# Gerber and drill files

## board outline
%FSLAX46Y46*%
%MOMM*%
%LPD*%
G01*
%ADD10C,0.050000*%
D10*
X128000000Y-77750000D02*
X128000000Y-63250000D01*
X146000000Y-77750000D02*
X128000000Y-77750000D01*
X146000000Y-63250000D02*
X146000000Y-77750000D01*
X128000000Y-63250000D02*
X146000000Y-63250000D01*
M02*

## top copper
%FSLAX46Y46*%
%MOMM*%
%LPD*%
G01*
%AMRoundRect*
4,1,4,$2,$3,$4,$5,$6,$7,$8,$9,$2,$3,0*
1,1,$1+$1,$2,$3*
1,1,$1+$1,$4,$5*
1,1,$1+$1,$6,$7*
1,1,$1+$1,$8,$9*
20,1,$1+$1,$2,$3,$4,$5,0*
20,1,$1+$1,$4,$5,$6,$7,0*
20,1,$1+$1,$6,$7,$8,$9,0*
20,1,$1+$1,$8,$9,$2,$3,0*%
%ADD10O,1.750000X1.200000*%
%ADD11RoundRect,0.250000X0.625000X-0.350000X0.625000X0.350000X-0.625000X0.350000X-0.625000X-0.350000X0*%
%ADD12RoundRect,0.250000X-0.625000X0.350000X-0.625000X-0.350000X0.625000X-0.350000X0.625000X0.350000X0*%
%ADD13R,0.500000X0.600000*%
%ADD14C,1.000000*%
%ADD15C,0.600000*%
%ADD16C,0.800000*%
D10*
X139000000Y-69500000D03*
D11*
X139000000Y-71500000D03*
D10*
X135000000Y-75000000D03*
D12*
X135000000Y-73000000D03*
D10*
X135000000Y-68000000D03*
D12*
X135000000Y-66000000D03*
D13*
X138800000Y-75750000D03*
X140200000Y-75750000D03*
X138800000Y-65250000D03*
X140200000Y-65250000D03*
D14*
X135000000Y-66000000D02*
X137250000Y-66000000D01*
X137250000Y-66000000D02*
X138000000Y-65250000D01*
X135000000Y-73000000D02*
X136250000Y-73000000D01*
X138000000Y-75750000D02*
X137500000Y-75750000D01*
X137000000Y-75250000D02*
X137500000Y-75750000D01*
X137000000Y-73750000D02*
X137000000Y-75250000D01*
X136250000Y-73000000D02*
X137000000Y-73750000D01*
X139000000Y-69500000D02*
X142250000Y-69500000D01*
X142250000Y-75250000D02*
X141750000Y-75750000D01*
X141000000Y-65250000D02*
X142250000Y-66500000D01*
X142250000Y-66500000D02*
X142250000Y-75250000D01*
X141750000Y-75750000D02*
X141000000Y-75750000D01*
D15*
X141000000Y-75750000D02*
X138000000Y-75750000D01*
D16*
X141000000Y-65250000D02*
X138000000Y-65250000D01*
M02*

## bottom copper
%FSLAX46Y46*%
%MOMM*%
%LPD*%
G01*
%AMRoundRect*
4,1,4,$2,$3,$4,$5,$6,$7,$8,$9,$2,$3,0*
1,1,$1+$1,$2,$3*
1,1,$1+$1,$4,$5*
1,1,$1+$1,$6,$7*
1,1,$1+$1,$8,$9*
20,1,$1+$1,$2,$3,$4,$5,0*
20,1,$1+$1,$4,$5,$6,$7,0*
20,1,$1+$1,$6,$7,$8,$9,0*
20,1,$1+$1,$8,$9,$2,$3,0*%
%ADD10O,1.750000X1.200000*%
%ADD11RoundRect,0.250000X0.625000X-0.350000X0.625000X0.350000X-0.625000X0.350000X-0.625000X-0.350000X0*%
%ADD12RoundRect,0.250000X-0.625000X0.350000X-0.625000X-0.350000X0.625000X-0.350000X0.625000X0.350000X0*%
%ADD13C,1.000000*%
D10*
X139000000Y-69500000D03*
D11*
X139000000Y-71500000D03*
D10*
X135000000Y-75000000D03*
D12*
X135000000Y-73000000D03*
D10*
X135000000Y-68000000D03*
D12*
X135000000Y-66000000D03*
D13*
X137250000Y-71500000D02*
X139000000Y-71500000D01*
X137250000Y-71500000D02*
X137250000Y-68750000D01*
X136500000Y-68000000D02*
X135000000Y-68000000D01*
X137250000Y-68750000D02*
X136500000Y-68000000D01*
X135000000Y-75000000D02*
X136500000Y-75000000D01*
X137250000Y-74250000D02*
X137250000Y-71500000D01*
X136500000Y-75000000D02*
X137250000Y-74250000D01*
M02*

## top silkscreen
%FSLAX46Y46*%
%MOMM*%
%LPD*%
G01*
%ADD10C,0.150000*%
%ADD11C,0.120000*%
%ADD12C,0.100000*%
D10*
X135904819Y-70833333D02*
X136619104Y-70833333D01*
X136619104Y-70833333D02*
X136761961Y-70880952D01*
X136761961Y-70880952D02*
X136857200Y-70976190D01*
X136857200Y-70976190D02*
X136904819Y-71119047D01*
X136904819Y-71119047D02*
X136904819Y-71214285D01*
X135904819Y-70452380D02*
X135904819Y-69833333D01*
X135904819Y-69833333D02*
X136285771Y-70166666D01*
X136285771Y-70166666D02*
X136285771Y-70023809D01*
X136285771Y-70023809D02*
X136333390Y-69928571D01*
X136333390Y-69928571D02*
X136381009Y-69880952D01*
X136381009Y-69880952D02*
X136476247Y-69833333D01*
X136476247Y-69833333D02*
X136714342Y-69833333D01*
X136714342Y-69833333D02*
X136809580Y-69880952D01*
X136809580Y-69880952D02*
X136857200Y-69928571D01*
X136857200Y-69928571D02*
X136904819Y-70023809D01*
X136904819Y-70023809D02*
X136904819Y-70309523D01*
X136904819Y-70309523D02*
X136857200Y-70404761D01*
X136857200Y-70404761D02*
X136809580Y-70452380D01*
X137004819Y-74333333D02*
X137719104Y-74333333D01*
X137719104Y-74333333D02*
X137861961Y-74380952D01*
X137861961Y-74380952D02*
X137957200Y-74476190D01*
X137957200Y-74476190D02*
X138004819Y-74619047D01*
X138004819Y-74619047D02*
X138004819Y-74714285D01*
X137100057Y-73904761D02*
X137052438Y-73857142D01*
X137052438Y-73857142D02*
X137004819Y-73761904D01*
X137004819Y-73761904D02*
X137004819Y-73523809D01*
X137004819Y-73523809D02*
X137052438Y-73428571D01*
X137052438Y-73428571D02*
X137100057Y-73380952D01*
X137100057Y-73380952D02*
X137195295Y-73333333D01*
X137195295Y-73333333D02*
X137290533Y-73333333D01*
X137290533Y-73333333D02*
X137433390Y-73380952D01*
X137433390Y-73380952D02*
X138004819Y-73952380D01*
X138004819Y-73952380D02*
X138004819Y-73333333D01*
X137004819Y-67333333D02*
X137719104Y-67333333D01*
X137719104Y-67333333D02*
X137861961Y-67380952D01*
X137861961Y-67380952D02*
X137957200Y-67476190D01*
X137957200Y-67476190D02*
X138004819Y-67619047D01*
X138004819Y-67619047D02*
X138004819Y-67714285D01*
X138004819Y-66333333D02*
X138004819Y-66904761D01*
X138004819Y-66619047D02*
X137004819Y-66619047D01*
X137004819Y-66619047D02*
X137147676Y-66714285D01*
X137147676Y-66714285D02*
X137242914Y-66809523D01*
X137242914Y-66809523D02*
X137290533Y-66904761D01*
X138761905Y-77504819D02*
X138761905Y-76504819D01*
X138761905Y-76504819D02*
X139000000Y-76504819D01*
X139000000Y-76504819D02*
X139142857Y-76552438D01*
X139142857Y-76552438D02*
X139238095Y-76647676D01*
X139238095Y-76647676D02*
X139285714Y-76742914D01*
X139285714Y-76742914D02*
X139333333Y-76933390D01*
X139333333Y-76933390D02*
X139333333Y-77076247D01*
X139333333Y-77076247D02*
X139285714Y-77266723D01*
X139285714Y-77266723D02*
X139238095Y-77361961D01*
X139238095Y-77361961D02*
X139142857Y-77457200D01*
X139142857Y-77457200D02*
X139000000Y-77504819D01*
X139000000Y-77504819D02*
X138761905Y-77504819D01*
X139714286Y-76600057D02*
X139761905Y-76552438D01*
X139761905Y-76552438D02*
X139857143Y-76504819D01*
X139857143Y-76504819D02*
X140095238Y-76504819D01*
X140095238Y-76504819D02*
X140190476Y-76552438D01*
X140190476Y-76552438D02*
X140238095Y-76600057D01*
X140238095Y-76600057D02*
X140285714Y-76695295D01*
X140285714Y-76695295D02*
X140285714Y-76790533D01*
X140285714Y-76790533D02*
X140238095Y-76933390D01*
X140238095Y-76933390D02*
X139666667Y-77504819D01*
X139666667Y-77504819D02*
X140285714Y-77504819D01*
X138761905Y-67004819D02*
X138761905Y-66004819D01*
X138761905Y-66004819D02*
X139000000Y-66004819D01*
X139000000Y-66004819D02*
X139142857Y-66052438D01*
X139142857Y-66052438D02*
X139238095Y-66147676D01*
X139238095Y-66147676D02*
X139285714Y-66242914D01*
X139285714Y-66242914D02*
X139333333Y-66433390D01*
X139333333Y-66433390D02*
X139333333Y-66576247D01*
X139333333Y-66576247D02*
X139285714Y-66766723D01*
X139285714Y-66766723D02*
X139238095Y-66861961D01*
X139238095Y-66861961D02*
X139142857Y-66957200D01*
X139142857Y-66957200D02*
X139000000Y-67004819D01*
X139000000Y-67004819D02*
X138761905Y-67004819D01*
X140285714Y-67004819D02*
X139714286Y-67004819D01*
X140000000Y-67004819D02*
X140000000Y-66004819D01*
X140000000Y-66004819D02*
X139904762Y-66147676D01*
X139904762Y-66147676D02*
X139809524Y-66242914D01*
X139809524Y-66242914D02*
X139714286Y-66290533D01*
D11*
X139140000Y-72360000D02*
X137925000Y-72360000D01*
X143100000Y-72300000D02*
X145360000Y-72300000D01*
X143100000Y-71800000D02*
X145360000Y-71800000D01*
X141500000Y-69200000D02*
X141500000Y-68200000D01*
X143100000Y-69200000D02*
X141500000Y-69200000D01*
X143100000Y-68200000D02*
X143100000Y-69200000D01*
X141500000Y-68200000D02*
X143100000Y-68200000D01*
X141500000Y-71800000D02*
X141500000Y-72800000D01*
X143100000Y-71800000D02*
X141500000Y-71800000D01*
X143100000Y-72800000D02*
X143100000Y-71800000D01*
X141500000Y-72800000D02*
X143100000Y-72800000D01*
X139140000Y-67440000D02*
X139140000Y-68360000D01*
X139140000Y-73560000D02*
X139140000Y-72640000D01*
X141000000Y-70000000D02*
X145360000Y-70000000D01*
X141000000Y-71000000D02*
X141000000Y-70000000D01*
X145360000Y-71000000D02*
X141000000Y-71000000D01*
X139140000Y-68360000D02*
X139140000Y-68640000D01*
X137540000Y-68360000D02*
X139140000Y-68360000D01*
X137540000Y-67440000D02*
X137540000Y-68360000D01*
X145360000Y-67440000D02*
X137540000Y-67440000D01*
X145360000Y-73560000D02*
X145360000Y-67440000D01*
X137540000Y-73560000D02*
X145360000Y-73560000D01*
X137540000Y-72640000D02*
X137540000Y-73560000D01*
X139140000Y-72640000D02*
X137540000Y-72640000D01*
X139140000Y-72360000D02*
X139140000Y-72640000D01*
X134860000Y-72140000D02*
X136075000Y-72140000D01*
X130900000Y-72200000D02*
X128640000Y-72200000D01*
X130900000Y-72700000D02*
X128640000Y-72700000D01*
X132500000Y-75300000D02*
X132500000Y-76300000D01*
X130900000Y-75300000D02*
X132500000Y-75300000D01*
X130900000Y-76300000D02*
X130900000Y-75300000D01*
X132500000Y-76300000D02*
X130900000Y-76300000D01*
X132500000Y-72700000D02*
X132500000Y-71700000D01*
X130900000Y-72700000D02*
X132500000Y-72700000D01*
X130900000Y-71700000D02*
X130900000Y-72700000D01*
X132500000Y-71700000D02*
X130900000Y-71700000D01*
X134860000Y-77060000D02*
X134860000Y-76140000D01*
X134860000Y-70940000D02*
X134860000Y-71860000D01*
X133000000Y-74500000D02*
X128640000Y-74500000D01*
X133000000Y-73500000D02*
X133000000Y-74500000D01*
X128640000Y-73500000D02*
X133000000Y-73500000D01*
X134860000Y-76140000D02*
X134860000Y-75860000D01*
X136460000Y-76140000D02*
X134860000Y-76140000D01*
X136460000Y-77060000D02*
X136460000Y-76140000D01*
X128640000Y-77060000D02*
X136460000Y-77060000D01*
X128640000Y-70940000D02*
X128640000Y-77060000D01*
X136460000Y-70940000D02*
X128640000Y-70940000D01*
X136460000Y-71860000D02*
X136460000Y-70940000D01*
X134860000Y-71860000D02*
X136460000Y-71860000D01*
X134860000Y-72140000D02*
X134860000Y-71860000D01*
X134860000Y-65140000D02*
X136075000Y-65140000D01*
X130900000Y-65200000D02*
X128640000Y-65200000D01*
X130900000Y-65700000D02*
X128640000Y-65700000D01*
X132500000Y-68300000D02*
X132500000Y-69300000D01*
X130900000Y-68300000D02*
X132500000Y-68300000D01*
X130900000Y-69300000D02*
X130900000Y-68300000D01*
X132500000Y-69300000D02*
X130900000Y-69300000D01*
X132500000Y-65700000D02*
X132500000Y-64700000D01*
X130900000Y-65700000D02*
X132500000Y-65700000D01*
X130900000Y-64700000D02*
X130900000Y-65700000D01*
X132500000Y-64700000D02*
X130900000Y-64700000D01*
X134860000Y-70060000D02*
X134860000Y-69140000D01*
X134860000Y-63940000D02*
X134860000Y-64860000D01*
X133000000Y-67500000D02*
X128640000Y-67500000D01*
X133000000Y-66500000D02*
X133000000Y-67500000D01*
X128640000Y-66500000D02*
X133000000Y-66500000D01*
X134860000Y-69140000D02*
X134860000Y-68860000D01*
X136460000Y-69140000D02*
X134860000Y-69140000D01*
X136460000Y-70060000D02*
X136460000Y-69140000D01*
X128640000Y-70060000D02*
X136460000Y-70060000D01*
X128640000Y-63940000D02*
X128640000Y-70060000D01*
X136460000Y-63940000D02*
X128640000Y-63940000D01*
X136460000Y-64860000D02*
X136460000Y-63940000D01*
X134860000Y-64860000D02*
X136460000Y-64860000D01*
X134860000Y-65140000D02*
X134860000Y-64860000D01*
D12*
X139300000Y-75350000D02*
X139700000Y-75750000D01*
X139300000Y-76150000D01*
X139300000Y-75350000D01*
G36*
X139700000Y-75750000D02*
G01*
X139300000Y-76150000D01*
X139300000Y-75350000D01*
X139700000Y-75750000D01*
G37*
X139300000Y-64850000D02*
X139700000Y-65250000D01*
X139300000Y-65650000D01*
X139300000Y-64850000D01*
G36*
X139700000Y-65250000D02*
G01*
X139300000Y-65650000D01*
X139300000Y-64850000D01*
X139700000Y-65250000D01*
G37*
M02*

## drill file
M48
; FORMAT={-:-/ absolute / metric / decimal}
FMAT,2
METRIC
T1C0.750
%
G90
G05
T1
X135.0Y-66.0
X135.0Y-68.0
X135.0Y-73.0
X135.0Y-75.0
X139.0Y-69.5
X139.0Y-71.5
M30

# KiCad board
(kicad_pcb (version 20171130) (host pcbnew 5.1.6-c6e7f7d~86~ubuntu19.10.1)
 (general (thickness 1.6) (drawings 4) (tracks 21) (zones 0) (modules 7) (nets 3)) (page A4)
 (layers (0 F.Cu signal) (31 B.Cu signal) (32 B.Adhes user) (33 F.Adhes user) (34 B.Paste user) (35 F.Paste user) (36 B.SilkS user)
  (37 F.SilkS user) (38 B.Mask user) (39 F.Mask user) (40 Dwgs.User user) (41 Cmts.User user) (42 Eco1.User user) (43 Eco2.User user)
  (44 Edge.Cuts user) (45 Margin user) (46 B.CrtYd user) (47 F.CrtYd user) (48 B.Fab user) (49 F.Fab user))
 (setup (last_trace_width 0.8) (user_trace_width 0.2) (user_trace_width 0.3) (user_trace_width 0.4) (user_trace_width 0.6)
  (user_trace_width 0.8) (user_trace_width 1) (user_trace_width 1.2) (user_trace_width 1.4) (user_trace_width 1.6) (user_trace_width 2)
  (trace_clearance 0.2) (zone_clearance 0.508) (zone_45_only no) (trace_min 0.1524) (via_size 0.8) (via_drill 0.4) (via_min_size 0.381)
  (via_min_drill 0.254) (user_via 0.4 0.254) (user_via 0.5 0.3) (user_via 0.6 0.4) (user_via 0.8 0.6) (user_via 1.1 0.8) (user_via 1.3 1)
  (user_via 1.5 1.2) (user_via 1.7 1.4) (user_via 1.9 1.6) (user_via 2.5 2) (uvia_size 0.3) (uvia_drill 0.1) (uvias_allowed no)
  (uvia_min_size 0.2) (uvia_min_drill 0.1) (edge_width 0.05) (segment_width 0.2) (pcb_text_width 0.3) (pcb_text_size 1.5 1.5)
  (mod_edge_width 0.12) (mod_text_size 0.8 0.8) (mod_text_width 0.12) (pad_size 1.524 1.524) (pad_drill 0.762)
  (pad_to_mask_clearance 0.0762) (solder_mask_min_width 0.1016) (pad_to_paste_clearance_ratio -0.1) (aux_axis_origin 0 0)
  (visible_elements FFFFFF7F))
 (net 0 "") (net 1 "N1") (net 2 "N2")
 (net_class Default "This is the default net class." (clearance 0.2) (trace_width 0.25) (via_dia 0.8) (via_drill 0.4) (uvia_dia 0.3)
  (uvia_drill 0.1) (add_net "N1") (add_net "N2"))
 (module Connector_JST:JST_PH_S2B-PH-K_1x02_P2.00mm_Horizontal (layer F.Cu) (at 139 71.5 90)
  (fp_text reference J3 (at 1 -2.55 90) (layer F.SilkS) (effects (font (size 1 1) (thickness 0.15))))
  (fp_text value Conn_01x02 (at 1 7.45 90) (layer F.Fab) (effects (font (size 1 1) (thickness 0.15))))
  (fp_line (start -0.86 0.14) (end -0.86 -1.075) (layer F.SilkS) (width 0.12))
  (fp_line (start -0.8 4.1) (end -0.8 6.36) (layer F.SilkS) (width 0.12))
  (fp_line (start -0.3 4.1) (end -0.3 6.36) (layer F.SilkS) (width 0.12))
  (fp_line (start 2.3 2.5) (end 3.3 2.5) (layer F.SilkS) (width 0.12))
  (fp_line (start 2.3 4.1) (end 2.3 2.5) (layer F.SilkS) (width 0.12))
  (fp_line (start 3.3 4.1) (end 2.3 4.1) (layer F.SilkS) (width 0.12))
  (fp_line (start 3.3 2.5) (end 3.3 4.1) (layer F.SilkS) (width 0.12))
  (fp_line (start -0.3 2.5) (end -1.3 2.5) (layer F.SilkS) (width 0.12))
  (fp_line (start -0.3 4.1) (end -0.3 2.5) (layer F.SilkS) (width 0.12))
  (fp_line (start -1.3 4.1) (end -0.3 4.1) (layer F.SilkS) (width 0.12))
  (fp_line (start -1.3 2.5) (end -1.3 4.1) (layer F.SilkS) (width 0.12))
  (fp_line (start 4.06 0.14) (end 3.14 0.14) (layer F.SilkS) (width 0.12))
  (fp_line (start -2.06 0.14) (end -1.14 0.14) (layer F.SilkS) (width 0.12))
  (fp_line (start 1.5 2) (end 1.5 6.36) (layer F.SilkS) (width 0.12))
  (fp_line (start 0.5 2) (end 1.5 2) (layer F.SilkS) (width 0.12))
  (fp_line (start 0.5 6.36) (end 0.5 2) (layer F.SilkS) (width 0.12))
  (fp_line (start 3.14 0.14) (end 2.86 0.14) (layer F.SilkS) (width 0.12))
  (fp_line (start 3.14 -1.46) (end 3.14 0.14) (layer F.SilkS) (width 0.12))
  (fp_line (start 4.06 -1.46) (end 3.14 -1.46) (layer F.SilkS) (width 0.12))
  (fp_line (start 4.06 6.36) (end 4.06 -1.46) (layer F.SilkS) (width 0.12))
  (fp_line (start -2.06 6.36) (end 4.06 6.36) (layer F.SilkS) (width 0.12))
  (fp_line (start -2.06 -1.46) (end -2.06 6.36) (layer F.SilkS) (width 0.12))
  (fp_line (start -1.14 -1.46) (end -2.06 -1.46) (layer F.SilkS) (width 0.12))
  (fp_line (start -1.14 0.14) (end -1.14 -1.46) (layer F.SilkS) (width 0.12))
  (fp_line (start -0.86 0.14) (end -1.14 0.14) (layer F.SilkS) (width 0.12))
  (pad 2 thru_hole oval (at 2 0 90) (size 1.2 1.75) (drill 0.75) (layers *.Cu *.Mask) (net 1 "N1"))
  (pad 1 thru_hole roundrect (at 0 0 90) (size 1.2 1.75) (drill 0.75) (layers *.Cu *.Mask) (roundrect_rratio 0.208333) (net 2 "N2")))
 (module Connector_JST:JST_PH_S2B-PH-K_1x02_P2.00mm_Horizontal (layer F.Cu) (at 135 73 270)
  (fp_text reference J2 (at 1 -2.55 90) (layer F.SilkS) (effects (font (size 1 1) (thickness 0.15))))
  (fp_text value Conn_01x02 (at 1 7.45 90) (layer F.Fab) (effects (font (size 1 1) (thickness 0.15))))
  (fp_line (start -0.86 0.14) (end -0.86 -1.075) (layer F.SilkS) (width 0.12))
  (fp_line (start -0.8 4.1) (end -0.8 6.36) (layer F.SilkS) (width 0.12))
  (fp_line (start -0.3 4.1) (end -0.3 6.36) (layer F.SilkS) (width 0.12))
  (fp_line (start 2.3 2.5) (end 3.3 2.5) (layer F.SilkS) (width 0.12))
  (fp_line (start 2.3 4.1) (end 2.3 2.5) (layer F.SilkS) (width 0.12))
  (fp_line (start 3.3 4.1) (end 2.3 4.1) (layer F.SilkS) (width 0.12))
  (fp_line (start 3.3 2.5) (end 3.3 4.1) (layer F.SilkS) (width 0.12))
  (fp_line (start -0.3 2.5) (end -1.3 2.5) (layer F.SilkS) (width 0.12))
  (fp_line (start -0.3 4.1) (end -0.3 2.5) (layer F.SilkS) (width 0.12))
  (fp_line (start -1.3 4.1) (end -0.3 4.1) (layer F.SilkS) (width 0.12))
  (fp_line (start -1.3 2.5) (end -1.3 4.1) (layer F.SilkS) (width 0.12))
  (fp_line (start 4.06 0.14) (end 3.14 0.14) (layer F.SilkS) (width 0.12))
  (fp_line (start -2.06 0.14) (end -1.14 0.14) (layer F.SilkS) (width 0.12))
  (fp_line (start 1.5 2) (end 1.5 6.36) (layer F.SilkS) (width 0.12))
  (fp_line (start 0.5 2) (end 1.5 2) (layer F.SilkS) (width 0.12))
  (fp_line (start 0.5 6.36) (end 0.5 2) (layer F.SilkS) (width 0.12))
  (fp_line (start 3.14 0.14) (end 2.86 0.14) (layer F.SilkS) (width 0.12))
  (fp_line (start 3.14 -1.46) (end 3.14 0.14) (layer F.SilkS) (width 0.12))
  (fp_line (start 4.06 -1.46) (end 3.14 -1.46) (layer F.SilkS) (width 0.12))
  (fp_line (start 4.06 6.36) (end 4.06 -1.46) (layer F.SilkS) (width 0.12))
  (fp_line (start -2.06 6.36) (end 4.06 6.36) (layer F.SilkS) (width 0.12))
  (fp_line (start -2.06 -1.46) (end -2.06 6.36) (layer F.SilkS) (width 0.12))
  (fp_line (start -1.14 -1.46) (end -2.06 -1.46) (layer F.SilkS) (width 0.12))
  (fp_line (start -1.14 0.14) (end -1.14 -1.46) (layer F.SilkS) (width 0.12))
  (fp_line (start -0.86 0.14) (end -1.14 0.14) (layer F.SilkS) (width 0.12))
  (pad 2 thru_hole oval (at 2 0 270) (size 1.2 1.75) (drill 0.75) (layers *.Cu *.Mask) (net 2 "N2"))
  (pad 1 thru_hole roundrect (at 0 0 270) (size 1.2 1.75) (drill 0.75) (layers *.Cu *.Mask) (roundrect_rratio 0.208333) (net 1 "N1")))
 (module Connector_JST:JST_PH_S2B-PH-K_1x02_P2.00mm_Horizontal (layer F.Cu) (at 135 66 270)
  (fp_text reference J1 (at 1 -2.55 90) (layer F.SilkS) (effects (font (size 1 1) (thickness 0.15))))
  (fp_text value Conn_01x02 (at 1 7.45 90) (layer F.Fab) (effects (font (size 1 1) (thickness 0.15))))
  (fp_line (start -0.86 0.14) (end -0.86 -1.075) (layer F.SilkS) (width 0.12))
  (fp_line (start -0.8 4.1) (end -0.8 6.36) (layer F.SilkS) (width 0.12))
  (fp_line (start -0.3 4.1) (end -0.3 6.36) (layer F.SilkS) (width 0.12))
  (fp_line (start 2.3 2.5) (end 3.3 2.5) (layer F.SilkS) (width 0.12))
  (fp_line (start 2.3 4.1) (end 2.3 2.5) (layer F.SilkS) (width 0.12))
  (fp_line (start 3.3 4.1) (end 2.3 4.1) (layer F.SilkS) (width 0.12))
  (fp_line (start 3.3 2.5) (end 3.3 4.1) (layer F.SilkS) (width 0.12))
  (fp_line (start -0.3 2.5) (end -1.3 2.5) (layer F.SilkS) (width 0.12))
  (fp_line (start -0.3 4.1) (end -0.3 2.5) (layer F.SilkS) (width 0.12))
  (fp_line (start -1.3 4.1) (end -0.3 4.1) (layer F.SilkS) (width 0.12))
  (fp_line (start -1.3 2.5) (end -1.3 4.1) (layer F.SilkS) (width 0.12))
  (fp_line (start 4.06 0.14) (end 3.14 0.14) (layer F.SilkS) (width 0.12))
  (fp_line (start -2.06 0.14) (end -1.14 0.14) (layer F.SilkS) (width 0.12))
  (fp_line (start 1.5 2) (end 1.5 6.36) (layer F.SilkS) (width 0.12))
  (fp_line (start 0.5 2) (end 1.5 2) (layer F.SilkS) (width 0.12))
  (fp_line (start 0.5 6.36) (end 0.5 2) (layer F.SilkS) (width 0.12))
  (fp_line (start 3.14 0.14) (end 2.86 0.14) (layer F.SilkS) (width 0.12))
  (fp_line (start 3.14 -1.46) (end 3.14 0.14) (layer F.SilkS) (width 0.12))
  (fp_line (start 4.06 -1.46) (end 3.14 -1.46) (layer F.SilkS) (width 0.12))
  (fp_line (start 4.06 6.36) (end 4.06 -1.46) (layer F.SilkS) (width 0.12))
  (fp_line (start -2.06 6.36) (end 4.06 6.36) (layer F.SilkS) (width 0.12))
  (fp_line (start -2.06 -1.46) (end -2.06 6.36) (layer F.SilkS) (width 0.12))
  (fp_line (start -1.14 -1.46) (end -2.06 -1.46) (layer F.SilkS) (width 0.12))
  (fp_line (start -1.14 0.14) (end -1.14 -1.46) (layer F.SilkS) (width 0.12))
  (fp_line (start -0.86 0.14) (end -1.14 0.14) (layer F.SilkS) (width 0.12))
  (pad 2 thru_hole oval (at 2 0 270) (size 1.2 1.75) (drill 0.75) (layers *.Cu *.Mask) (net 2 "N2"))
  (pad 1 thru_hole roundrect (at 0 0 270) (size 1.2 1.75) (drill 0.75) (layers *.Cu *.Mask) (roundrect_rratio 0.208333) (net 1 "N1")))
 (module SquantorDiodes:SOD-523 (layer F.Cu) (at 139.5 75.75 180)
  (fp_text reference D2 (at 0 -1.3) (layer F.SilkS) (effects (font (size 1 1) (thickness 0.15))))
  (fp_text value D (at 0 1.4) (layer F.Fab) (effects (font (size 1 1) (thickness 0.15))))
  (fp_poly (pts (xy 0.2 0.4) (xy -0.2 0) (xy 0.2 -0.4)) (layer F.SilkS) (width 0.1))
  (pad 2 smd rect (at 0.7 0 180) (size 0.5 0.6) (layers F.Cu F.Paste F.Mask) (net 1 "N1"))
  (pad 1 smd rect (at -0.7 0 180) (size 0.5 0.6) (layers F.Cu F.Paste F.Mask) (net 1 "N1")))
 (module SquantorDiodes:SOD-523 (layer F.Cu) (at 139.5 65.25 180)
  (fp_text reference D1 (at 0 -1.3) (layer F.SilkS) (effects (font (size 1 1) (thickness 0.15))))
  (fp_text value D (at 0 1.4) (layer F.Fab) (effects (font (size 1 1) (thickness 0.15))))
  (fp_poly (pts (xy 0.2 0.4) (xy -0.2 0) (xy 0.2 -0.4)) (layer F.SilkS) (width 0.1))
  (pad 2 smd rect (at 0.7 0 180) (size 0.5 0.6) (layers F.Cu F.Paste F.Mask) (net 1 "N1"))
  (pad 1 smd rect (at -0.7 0 180) (size 0.5 0.6) (layers F.Cu F.Paste F.Mask) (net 1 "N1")))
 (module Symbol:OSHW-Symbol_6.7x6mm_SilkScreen (layer B.Cu) (at 142.3 66.35 180)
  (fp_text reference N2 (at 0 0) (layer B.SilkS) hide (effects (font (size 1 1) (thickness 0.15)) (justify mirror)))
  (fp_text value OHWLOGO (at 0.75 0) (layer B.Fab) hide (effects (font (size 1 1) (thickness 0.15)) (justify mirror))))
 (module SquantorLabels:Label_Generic (layer B.Cu) (at 143.25 73 180)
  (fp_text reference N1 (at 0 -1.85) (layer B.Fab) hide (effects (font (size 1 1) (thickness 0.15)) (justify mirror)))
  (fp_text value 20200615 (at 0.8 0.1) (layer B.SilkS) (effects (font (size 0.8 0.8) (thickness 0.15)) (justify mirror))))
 (gr_line (start 128 77.75) (end 128 63.25) (layer Edge.Cuts) (width 0.05))
 (gr_line (start 146 77.75) (end 128 77.75) (layer Edge.Cuts) (width 0.05))
 (gr_line (start 146 63.25) (end 146 77.75) (layer Edge.Cuts) (width 0.05))
 (gr_line (start 128 63.25) (end 146 63.25) (layer Edge.Cuts) (width 0.05))
 (segment (start 135 66) (end 137.25 66) (width 1) (layer F.Cu) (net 1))
 (segment (start 137.25 66) (end 138 65.25) (width 1) (layer F.Cu) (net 1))
 (segment (start 135 73) (end 136.25 73) (width 1) (layer F.Cu) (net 1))
 (segment (start 138 75.75) (end 137.5 75.75) (width 1) (layer F.Cu) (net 1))
 (segment (start 137 75.25) (end 137.5 75.75) (width 1) (layer F.Cu) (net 1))
 (segment (start 137 73.75) (end 137 75.25) (width 1) (layer F.Cu) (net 1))
 (segment (start 136.25 73) (end 137 73.75) (width 1) (layer F.Cu) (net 1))
 (segment (start 139 69.5) (end 142.25 69.5) (width 1) (layer F.Cu) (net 1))
 (segment (start 142.25 75.25) (end 141.75 75.75) (width 1) (layer F.Cu) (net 1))
 (segment (start 141 65.25) (end 142.25 66.5) (width 1) (layer F.Cu) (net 1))
 (segment (start 142.25 66.5) (end 142.25 75.25) (width 1) (layer F.Cu) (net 1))
 (segment (start 141.75 75.75) (end 141 75.75) (width 1) (layer F.Cu) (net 1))
 (segment (start 141 75.75) (end 138 75.75) (width 0.6) (layer F.Cu) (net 1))
 (segment (start 141 65.25) (end 138 65.25) (width 0.8) (layer F.Cu) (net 1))
 (segment (start 137.25 71.5) (end 139 71.5) (width 1) (layer B.Cu) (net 2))
 (segment (start 137.25 71.5) (end 137.25 68.75) (width 1) (layer B.Cu) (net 2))
 (segment (start 136.5 68) (end 135 68) (width 1) (layer B.Cu) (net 2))
 (segment (start 137.25 68.75) (end 136.5 68) (width 1) (layer B.Cu) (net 2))
 (segment (start 135 75) (end 136.5 75) (width 1) (layer B.Cu) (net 2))
 (segment (start 137.25 74.25) (end 137.25 71.5) (width 1) (layer B.Cu) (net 2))
 (segment (start 136.5 75) (end 137.25 74.25) (width 1) (layer B.Cu) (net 2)))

